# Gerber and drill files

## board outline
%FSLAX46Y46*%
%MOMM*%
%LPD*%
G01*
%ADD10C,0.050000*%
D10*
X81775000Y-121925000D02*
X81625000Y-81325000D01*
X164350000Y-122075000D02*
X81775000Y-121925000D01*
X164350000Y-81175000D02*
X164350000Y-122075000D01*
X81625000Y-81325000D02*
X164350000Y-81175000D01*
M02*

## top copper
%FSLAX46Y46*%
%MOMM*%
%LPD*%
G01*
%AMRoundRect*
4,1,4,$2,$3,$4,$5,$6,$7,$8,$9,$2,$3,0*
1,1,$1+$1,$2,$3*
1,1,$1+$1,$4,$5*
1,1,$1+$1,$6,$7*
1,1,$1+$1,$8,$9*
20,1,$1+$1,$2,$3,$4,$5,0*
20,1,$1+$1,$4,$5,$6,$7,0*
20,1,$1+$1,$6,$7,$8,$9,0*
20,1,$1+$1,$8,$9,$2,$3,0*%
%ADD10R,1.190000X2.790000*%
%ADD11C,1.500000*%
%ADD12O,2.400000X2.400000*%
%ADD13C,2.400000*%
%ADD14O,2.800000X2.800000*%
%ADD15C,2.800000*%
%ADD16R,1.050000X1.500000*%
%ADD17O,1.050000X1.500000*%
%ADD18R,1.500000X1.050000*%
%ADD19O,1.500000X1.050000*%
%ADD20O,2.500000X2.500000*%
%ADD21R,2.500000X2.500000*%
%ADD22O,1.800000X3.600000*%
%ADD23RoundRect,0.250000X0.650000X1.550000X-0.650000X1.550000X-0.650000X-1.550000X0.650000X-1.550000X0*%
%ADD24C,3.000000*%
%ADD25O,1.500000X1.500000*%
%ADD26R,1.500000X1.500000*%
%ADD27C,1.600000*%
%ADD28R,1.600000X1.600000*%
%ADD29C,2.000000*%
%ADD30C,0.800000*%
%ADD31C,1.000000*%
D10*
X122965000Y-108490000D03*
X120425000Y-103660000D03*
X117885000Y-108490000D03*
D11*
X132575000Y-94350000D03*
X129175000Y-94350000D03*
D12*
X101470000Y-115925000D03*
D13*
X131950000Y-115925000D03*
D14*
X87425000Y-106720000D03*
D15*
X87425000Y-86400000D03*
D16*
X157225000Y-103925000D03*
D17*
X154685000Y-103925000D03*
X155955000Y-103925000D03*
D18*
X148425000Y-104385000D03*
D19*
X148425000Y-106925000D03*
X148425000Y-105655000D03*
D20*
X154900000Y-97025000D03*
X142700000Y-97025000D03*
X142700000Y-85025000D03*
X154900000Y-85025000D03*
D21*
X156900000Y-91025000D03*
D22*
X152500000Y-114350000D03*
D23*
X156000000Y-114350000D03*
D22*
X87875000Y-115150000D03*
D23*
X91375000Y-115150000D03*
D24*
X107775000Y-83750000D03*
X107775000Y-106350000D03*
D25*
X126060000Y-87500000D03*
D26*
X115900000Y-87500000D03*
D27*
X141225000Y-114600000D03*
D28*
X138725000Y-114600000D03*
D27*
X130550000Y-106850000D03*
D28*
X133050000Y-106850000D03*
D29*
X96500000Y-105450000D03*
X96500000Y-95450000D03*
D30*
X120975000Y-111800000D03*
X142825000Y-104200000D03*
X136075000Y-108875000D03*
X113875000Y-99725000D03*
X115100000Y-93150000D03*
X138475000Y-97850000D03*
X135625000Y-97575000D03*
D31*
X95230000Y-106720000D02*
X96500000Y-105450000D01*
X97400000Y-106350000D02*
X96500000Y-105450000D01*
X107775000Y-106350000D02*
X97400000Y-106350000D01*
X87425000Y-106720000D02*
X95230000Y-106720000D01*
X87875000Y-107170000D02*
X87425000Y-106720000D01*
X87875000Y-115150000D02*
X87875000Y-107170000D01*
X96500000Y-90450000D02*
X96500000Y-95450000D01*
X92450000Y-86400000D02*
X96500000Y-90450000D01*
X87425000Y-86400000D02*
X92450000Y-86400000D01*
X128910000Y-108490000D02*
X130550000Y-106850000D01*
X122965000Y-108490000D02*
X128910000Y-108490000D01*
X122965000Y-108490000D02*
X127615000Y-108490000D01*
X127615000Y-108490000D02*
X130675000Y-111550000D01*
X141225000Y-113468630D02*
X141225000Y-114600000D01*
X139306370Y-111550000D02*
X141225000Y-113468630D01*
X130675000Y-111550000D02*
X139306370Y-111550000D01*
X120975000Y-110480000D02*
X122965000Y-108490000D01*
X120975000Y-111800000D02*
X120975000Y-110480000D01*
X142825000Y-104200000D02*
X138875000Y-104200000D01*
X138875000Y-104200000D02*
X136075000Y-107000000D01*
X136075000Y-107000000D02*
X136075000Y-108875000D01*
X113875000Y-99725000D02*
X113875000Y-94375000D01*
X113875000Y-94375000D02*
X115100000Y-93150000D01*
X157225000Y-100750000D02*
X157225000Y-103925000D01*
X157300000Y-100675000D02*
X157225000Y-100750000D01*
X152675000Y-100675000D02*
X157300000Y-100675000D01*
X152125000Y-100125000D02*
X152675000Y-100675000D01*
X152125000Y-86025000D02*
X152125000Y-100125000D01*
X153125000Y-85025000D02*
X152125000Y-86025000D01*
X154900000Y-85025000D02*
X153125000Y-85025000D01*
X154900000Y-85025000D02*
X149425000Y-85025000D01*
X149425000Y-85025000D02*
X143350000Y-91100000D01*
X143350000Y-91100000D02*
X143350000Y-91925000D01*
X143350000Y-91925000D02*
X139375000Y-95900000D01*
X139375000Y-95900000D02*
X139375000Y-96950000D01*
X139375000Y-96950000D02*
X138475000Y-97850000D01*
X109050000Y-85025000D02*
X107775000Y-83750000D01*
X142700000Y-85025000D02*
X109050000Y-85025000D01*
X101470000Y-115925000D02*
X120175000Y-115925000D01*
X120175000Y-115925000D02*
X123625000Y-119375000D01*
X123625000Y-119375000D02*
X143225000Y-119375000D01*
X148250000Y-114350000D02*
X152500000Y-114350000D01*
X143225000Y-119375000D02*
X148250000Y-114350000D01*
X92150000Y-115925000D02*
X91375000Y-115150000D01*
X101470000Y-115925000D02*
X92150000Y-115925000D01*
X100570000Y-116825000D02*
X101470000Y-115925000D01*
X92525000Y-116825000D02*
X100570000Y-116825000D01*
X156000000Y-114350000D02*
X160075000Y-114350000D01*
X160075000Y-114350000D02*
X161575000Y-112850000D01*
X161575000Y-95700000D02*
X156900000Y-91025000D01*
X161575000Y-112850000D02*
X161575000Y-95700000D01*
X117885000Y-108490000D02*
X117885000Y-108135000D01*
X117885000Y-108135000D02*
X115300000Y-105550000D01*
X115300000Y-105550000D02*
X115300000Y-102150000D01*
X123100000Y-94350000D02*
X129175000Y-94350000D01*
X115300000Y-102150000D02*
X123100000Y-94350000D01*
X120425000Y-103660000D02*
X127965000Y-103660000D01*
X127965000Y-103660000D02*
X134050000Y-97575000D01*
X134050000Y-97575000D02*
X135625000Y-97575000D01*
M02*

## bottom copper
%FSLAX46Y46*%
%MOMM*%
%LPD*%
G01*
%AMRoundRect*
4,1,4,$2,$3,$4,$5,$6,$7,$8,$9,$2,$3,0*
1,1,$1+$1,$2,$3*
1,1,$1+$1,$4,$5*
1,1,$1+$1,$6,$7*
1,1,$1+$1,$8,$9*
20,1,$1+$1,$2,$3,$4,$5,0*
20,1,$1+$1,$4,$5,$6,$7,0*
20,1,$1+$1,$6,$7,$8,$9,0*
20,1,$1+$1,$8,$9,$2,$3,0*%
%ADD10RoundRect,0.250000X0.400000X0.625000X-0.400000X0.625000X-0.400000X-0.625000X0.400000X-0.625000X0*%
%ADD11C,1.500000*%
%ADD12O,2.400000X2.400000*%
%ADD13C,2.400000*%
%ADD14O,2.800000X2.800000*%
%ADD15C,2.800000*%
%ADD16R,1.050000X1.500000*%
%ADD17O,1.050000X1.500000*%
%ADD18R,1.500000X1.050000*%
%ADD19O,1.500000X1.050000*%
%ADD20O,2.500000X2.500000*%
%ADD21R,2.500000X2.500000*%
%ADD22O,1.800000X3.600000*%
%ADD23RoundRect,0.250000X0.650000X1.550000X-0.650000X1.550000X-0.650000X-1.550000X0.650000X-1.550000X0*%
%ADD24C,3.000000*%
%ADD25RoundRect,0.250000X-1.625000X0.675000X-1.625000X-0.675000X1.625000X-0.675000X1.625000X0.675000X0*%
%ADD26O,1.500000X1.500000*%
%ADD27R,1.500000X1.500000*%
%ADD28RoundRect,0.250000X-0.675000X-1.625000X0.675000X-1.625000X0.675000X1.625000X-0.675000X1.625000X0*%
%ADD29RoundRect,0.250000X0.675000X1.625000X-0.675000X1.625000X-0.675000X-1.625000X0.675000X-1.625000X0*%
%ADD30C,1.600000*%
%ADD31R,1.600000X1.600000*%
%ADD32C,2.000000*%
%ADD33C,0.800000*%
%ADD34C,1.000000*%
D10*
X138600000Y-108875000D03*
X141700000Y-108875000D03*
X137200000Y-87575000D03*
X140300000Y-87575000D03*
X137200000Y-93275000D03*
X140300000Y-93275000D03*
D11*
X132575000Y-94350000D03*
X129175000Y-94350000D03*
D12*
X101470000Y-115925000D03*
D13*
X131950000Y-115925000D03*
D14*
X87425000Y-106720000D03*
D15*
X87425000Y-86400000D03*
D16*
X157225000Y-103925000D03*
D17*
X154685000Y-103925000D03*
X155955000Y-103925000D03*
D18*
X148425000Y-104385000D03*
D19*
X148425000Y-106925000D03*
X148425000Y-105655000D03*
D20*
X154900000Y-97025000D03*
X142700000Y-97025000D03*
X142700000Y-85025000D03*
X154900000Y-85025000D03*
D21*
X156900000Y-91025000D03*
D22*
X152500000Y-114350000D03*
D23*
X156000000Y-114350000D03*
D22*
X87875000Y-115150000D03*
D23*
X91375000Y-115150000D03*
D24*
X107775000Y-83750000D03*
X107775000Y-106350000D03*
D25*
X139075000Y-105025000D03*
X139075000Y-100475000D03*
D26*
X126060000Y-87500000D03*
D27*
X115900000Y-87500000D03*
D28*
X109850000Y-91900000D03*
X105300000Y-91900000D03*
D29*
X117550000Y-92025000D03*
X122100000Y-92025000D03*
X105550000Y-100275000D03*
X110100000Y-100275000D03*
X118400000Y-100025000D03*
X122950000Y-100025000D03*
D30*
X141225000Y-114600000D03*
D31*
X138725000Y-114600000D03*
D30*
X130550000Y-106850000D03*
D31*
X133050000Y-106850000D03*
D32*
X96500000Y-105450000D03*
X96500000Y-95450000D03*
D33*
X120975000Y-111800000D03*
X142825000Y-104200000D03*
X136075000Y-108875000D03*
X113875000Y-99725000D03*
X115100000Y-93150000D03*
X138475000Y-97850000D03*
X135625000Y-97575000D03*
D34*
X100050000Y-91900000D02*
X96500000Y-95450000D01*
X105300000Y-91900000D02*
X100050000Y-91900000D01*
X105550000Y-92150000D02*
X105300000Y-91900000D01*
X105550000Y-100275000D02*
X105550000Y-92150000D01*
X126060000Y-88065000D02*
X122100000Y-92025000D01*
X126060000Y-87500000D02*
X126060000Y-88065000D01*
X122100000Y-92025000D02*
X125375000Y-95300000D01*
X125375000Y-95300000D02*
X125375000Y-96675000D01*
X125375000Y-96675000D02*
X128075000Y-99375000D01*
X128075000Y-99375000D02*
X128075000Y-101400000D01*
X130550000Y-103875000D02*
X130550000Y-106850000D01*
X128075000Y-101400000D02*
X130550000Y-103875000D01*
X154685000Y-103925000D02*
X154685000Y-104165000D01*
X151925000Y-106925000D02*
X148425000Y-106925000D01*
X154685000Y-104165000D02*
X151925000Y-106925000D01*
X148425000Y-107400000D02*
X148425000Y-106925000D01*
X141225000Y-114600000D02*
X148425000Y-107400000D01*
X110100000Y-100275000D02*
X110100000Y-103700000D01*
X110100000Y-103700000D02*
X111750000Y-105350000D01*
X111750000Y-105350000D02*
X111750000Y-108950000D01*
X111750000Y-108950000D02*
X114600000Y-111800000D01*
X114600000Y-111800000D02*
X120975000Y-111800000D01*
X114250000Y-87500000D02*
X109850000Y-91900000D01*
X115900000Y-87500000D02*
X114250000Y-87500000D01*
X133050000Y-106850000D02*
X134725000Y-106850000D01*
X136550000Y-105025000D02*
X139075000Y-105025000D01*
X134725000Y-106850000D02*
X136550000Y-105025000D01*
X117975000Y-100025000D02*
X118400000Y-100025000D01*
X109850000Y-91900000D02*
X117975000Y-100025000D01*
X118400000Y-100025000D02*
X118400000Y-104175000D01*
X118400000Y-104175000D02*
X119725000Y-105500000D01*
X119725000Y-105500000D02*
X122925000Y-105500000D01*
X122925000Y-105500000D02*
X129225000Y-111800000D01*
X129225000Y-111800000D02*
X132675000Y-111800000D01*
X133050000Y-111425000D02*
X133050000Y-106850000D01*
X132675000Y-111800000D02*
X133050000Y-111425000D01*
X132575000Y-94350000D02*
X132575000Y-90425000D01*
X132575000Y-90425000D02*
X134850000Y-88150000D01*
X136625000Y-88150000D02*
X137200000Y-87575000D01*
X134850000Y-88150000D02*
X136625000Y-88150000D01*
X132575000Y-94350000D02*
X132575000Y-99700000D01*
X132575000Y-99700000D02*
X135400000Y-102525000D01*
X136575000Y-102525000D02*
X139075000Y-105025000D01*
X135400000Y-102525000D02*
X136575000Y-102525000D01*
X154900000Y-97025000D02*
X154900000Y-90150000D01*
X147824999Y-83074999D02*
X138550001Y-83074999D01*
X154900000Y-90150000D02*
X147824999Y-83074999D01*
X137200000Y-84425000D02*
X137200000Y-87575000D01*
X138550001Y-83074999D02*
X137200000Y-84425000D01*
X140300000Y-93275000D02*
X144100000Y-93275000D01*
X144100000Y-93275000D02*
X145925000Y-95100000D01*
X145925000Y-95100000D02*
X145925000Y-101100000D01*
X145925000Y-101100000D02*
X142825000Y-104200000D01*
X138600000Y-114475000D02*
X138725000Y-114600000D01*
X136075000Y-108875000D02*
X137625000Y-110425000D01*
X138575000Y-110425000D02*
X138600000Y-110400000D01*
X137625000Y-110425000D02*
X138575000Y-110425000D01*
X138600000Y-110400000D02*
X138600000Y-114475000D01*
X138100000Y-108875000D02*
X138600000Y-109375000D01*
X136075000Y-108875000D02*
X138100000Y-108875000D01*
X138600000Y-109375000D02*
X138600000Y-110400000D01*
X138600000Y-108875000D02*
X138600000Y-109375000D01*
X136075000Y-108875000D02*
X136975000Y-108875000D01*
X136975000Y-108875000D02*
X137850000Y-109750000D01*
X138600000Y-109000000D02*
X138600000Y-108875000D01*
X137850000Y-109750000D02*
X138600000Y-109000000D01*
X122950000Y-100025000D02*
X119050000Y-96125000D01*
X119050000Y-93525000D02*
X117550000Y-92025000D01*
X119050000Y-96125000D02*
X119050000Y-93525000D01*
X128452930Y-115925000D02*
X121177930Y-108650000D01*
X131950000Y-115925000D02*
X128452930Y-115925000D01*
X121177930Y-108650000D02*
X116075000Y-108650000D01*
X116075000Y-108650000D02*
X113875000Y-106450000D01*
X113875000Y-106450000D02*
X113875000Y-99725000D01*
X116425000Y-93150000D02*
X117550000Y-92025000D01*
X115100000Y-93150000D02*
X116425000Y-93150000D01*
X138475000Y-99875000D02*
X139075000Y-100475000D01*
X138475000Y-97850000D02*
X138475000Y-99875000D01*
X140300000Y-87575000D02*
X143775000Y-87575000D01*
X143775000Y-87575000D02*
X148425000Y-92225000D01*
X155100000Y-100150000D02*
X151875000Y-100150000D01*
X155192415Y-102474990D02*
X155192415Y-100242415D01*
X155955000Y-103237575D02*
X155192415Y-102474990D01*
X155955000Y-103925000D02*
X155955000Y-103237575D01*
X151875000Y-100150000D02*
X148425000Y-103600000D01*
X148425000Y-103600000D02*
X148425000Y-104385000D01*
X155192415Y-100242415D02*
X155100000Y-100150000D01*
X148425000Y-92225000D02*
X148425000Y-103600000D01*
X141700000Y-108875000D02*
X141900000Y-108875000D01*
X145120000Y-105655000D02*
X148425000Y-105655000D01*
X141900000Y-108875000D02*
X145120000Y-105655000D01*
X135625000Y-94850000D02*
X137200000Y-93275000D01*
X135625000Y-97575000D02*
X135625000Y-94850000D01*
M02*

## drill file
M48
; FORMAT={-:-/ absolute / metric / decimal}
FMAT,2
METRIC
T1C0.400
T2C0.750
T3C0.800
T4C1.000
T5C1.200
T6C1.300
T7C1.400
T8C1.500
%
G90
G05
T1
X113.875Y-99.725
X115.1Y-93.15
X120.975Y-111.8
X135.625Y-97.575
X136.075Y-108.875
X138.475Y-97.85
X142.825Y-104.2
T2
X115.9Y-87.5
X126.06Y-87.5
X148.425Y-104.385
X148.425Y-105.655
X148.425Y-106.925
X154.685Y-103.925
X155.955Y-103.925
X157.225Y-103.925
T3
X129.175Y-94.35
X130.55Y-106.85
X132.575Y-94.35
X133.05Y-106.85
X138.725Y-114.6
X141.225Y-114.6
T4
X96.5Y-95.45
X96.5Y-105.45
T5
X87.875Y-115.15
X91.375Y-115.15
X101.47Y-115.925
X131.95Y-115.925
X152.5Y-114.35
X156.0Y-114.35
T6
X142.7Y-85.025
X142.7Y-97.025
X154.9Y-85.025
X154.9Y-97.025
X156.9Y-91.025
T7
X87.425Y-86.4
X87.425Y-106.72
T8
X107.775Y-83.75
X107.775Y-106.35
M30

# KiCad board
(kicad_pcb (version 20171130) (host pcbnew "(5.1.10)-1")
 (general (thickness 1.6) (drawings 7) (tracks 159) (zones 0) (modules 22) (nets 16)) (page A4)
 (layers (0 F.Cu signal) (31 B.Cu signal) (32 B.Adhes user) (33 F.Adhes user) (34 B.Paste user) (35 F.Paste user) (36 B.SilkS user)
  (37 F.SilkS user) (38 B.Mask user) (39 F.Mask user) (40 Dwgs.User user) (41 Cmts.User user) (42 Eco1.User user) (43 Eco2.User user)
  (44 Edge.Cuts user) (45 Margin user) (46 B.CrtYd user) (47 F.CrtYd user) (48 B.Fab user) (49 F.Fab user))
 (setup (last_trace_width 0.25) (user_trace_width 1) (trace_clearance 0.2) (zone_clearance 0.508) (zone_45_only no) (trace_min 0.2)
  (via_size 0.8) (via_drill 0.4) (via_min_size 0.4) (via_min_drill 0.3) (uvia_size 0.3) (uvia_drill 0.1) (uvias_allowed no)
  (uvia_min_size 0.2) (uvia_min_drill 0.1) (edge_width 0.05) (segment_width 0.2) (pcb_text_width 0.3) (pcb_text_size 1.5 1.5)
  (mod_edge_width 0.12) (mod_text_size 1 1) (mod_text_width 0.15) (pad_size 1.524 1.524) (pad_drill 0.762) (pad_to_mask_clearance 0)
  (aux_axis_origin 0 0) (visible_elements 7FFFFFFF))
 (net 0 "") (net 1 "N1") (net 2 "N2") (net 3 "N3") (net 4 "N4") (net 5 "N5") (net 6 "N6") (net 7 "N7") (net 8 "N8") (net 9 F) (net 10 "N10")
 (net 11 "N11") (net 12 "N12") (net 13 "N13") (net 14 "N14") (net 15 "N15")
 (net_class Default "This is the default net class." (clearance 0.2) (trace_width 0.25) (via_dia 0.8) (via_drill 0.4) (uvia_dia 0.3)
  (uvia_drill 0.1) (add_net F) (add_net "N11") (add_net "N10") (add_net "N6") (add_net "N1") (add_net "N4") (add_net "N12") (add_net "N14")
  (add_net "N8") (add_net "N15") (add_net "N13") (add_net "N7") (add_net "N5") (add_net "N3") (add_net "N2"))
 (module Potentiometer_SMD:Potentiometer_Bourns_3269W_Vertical (layer F.Cu) (at 120.425 106.075 180)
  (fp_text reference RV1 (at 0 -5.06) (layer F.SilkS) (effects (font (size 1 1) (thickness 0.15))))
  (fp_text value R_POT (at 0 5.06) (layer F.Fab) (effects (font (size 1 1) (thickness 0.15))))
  (pad 3 smd rect (at -2.54 -2.415 180) (size 1.19 2.79) (layers F.Cu F.Paste F.Mask) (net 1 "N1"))
  (pad 2 smd rect (at 0 2.415 180) (size 1.19 2.79) (layers F.Cu F.Paste F.Mask) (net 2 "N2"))
  (pad 1 smd rect (at 2.54 -2.415 180) (size 1.19 2.79) (layers F.Cu F.Paste F.Mask) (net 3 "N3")))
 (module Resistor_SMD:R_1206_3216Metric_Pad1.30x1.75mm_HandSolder (layer B.Cu) (at 140.15 108.875 180)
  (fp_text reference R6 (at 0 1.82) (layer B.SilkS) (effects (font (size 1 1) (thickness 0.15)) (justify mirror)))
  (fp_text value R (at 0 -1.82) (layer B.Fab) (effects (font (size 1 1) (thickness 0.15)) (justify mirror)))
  (pad 2 smd roundrect (at 1.55 0 180) (size 1.3 1.75) (layers B.Cu B.Paste B.Mask) (roundrect_rratio 0.192308) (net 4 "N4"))
  (pad 1 smd roundrect (at -1.55 0 180) (size 1.3 1.75) (layers B.Cu B.Paste B.Mask) (roundrect_rratio 0.192308) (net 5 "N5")))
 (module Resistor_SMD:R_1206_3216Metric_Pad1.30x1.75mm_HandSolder (layer B.Cu) (at 138.75 87.575 180)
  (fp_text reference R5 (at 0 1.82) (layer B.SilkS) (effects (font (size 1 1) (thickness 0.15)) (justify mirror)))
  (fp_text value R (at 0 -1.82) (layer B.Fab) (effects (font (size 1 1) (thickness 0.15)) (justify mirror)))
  (pad 2 smd roundrect (at 1.55 0 180) (size 1.3 1.75) (layers B.Cu B.Paste B.Mask) (roundrect_rratio 0.192308) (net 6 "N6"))
  (pad 1 smd roundrect (at -1.55 0 180) (size 1.3 1.75) (layers B.Cu B.Paste B.Mask) (roundrect_rratio 0.192308) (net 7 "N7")))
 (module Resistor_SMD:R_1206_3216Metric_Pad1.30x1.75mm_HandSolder (layer B.Cu) (at 138.75 93.275 180)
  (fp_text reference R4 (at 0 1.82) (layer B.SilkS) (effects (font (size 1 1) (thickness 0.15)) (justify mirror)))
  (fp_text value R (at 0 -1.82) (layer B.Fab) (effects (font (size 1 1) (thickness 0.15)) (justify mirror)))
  (pad 2 smd roundrect (at 1.55 0 180) (size 1.3 1.75) (layers B.Cu B.Paste B.Mask) (roundrect_rratio 0.192308) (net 2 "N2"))
  (pad 1 smd roundrect (at -1.55 0 180) (size 1.3 1.75) (layers B.Cu B.Paste B.Mask) (roundrect_rratio 0.192308) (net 4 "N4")))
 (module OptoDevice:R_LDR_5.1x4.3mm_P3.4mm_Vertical (layer F.Cu) (at 129.175 94.35)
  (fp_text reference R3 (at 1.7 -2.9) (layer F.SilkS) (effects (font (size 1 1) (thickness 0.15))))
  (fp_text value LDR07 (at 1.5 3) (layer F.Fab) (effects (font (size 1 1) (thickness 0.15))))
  (pad 2 thru_hole circle (at 3.4 0) (size 1.5 1.5) (drill 0.8) (layers *.Cu *.Mask) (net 6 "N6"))
  (pad 1 thru_hole circle (at 0 0) (size 1.5 1.5) (drill 0.8) (layers *.Cu *.Mask) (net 3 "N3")))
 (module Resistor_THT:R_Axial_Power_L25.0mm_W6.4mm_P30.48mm (layer F.Cu) (at 131.95 115.925 180)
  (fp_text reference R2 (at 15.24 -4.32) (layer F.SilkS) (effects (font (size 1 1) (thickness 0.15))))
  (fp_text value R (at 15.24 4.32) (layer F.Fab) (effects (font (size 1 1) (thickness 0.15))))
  (pad 2 thru_hole oval (at 30.48 0 180) (size 2.4 2.4) (drill 1.2) (layers *.Cu *.Mask) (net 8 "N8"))
  (pad 1 thru_hole circle (at 0 0 180) (size 2.4 2.4) (drill 1.2) (layers *.Cu *.Mask) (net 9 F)))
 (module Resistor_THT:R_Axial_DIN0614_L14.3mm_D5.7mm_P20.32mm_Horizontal (layer F.Cu) (at 87.425 86.4 270)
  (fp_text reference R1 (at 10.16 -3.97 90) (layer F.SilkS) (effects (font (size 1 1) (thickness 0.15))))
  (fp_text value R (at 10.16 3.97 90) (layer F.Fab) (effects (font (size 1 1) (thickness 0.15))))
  (pad 2 thru_hole oval (at 20.32 0 270) (size 2.8 2.8) (drill 1.4) (layers *.Cu *.Mask) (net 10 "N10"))
  (pad 1 thru_hole circle (at 0 0 270) (size 2.8 2.8) (drill 1.4) (layers *.Cu *.Mask) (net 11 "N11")))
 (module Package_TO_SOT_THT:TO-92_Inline (layer F.Cu) (at 157.225 103.925 180)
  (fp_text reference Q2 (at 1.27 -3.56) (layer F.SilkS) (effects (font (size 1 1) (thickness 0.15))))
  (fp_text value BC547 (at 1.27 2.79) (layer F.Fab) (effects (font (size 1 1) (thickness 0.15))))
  (pad 1 thru_hole rect (at 0 0 180) (size 1.05 1.5) (drill 0.75) (layers *.Cu *.Mask) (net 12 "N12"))
  (pad 3 thru_hole oval (at 2.54 0 180) (size 1.05 1.5) (drill 0.75) (layers *.Cu *.Mask) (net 1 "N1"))
  (pad 2 thru_hole oval (at 1.27 0 180) (size 1.05 1.5) (drill 0.75) (layers *.Cu *.Mask) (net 7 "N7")))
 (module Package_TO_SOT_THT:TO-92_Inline (layer F.Cu) (at 148.425 104.385 270)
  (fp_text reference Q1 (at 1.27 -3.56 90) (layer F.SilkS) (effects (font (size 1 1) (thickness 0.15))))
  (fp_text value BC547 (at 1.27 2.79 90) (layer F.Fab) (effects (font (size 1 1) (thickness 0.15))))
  (pad 1 thru_hole rect (at 0 0 270) (size 1.05 1.5) (drill 0.75) (layers *.Cu *.Mask) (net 7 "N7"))
  (pad 3 thru_hole oval (at 2.54 0 270) (size 1.05 1.5) (drill 0.75) (layers *.Cu *.Mask) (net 1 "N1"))
  (pad 2 thru_hole oval (at 1.27 0 270) (size 1.05 1.5) (drill 0.75) (layers *.Cu *.Mask) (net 5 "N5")))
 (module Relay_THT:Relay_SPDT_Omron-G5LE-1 (layer F.Cu) (at 156.9 91.025 270)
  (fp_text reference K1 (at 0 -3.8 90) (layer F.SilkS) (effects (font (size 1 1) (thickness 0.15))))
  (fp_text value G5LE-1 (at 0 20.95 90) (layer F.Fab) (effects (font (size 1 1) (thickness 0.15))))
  (pad 5 thru_hole oval (at 6 2 270) (size 2.5 2.5) (drill 1.3) (layers *.Cu *.Mask) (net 6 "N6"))
  (pad 4 thru_hole oval (at 6 14.2 270) (size 2.5 2.5) (drill 1.3) (layers *.Cu *.Mask) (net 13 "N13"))
  (pad 3 thru_hole oval (at -6 14.2 270) (size 2.5 2.5) (drill 1.3) (layers *.Cu *.Mask) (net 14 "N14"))
  (pad 2 thru_hole oval (at -6 2 270) (size 2.5 2.5) (drill 1.3) (layers *.Cu *.Mask) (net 12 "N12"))
  (pad 1 thru_hole rect (at 0 0 270) (size 2.5 2.5) (drill 1.3) (layers *.Cu *.Mask) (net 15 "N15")))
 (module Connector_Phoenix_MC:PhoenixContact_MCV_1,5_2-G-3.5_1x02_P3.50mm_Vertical (layer F.Cu) (at 156 114.35 180)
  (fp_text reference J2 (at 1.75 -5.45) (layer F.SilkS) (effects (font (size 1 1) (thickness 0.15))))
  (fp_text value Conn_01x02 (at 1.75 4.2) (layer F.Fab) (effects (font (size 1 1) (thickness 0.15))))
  (pad 2 thru_hole oval (at 3.5 0 180) (size 1.8 3.6) (drill 1.2) (layers *.Cu *.Mask) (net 8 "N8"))
  (pad 1 thru_hole roundrect (at 0 0 180) (size 1.8 3.6) (drill 1.2) (layers *.Cu *.Mask) (roundrect_rratio 0.138889) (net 15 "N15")))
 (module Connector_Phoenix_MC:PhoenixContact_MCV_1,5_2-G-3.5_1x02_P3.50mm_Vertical (layer F.Cu) (at 91.375 115.15 180)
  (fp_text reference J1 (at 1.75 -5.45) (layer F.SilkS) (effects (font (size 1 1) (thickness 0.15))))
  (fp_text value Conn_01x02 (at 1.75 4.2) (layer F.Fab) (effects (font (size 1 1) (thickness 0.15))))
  (pad 2 thru_hole oval (at 3.5 0 180) (size 1.8 3.6) (drill 1.2) (layers *.Cu *.Mask) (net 10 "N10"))
  (pad 1 thru_hole roundrect (at 0 0 180) (size 1.8 3.6) (drill 1.2) (layers *.Cu *.Mask) (roundrect_rratio 0.138889) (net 8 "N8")))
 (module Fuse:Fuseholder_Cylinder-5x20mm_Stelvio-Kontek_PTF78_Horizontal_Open (layer F.Cu) (at 107.775 83.75 270)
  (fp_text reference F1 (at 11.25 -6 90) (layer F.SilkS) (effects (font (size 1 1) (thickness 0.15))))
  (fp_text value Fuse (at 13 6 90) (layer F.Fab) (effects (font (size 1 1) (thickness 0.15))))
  (pad 1 thru_hole circle (at 0 0 270) (size 3 3) (drill 1.5) (layers *.Cu *.Mask) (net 14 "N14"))
  (pad 2 thru_hole circle (at 22.6 0 270) (size 3 3) (drill 1.5) (layers *.Cu *.Mask) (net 10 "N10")))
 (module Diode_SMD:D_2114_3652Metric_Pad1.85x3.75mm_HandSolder (layer B.Cu) (at 139.075 102.75 270)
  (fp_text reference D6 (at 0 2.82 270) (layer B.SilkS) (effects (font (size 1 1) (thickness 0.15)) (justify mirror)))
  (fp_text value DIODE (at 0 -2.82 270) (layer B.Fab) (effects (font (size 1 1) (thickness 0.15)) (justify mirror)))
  (pad 2 smd roundrect (at 2.275 0 270) (size 1.85 3.75) (layers B.Cu B.Paste B.Mask) (roundrect_rratio 0.135135) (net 6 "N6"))
  (pad 1 smd roundrect (at -2.275 0 270) (size 1.85 3.75) (layers B.Cu B.Paste B.Mask) (roundrect_rratio 0.135135) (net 12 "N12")))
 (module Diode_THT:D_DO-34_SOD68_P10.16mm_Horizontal (layer F.Cu) (at 115.9 87.5)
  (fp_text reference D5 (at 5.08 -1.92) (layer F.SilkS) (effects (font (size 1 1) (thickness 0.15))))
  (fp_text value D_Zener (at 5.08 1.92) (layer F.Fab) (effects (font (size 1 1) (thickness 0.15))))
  (pad 2 thru_hole oval (at 10.16 0) (size 1.5 1.5) (drill 0.75) (layers *.Cu *.Mask) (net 1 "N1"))
  (pad 1 thru_hole rect (at 0 0) (size 1.5 1.5) (drill 0.75) (layers *.Cu *.Mask) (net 6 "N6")))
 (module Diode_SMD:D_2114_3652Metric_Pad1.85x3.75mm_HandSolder (layer B.Cu) (at 107.575 91.9)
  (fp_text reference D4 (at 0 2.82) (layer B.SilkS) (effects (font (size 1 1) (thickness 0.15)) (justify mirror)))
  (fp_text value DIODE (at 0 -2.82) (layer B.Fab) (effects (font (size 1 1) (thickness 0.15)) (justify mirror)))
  (pad 2 smd roundrect (at 2.275 0) (size 1.85 3.75) (layers B.Cu B.Paste B.Mask) (roundrect_rratio 0.135135) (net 6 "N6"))
  (pad 1 smd roundrect (at -2.275 0) (size 1.85 3.75) (layers B.Cu B.Paste B.Mask) (roundrect_rratio 0.135135) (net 11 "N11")))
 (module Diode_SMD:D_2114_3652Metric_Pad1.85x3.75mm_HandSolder (layer B.Cu) (at 119.825 92.025 180)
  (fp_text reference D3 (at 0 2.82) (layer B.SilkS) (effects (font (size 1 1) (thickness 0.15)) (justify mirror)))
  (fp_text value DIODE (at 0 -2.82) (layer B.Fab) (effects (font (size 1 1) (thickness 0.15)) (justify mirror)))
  (pad 2 smd roundrect (at 2.275 0 180) (size 1.85 3.75) (layers B.Cu B.Paste B.Mask) (roundrect_rratio 0.135135) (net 9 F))
  (pad 1 smd roundrect (at -2.275 0 180) (size 1.85 3.75) (layers B.Cu B.Paste B.Mask) (roundrect_rratio 0.135135) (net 1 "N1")))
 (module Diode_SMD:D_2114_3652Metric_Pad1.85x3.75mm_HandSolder (layer B.Cu) (at 107.825 100.275 180)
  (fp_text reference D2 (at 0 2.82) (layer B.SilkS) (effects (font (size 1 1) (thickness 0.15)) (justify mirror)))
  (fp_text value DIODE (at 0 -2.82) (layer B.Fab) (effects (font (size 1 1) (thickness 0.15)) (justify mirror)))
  (pad 2 smd roundrect (at 2.275 0 180) (size 1.85 3.75) (layers B.Cu B.Paste B.Mask) (roundrect_rratio 0.135135) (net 11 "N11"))
  (pad 1 smd roundrect (at -2.275 0 180) (size 1.85 3.75) (layers B.Cu B.Paste B.Mask) (roundrect_rratio 0.135135) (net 1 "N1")))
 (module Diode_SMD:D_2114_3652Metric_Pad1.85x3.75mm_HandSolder (layer B.Cu) (at 120.675 100.025 180)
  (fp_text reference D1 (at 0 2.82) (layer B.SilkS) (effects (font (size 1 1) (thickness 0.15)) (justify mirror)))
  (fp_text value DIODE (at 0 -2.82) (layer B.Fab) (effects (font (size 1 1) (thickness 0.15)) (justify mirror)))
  (pad 2 smd roundrect (at 2.275 0 180) (size 1.85 3.75) (layers B.Cu B.Paste B.Mask) (roundrect_rratio 0.135135) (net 6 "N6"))
  (pad 1 smd roundrect (at -2.275 0 180) (size 1.85 3.75) (layers B.Cu B.Paste B.Mask) (roundrect_rratio 0.135135) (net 9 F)))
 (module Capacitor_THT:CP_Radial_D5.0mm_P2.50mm (layer F.Cu) (at 138.725 114.6)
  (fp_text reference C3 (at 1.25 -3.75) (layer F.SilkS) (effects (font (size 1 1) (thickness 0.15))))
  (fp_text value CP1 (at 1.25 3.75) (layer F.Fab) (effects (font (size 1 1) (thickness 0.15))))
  (pad 2 thru_hole circle (at 2.5 0) (size 1.6 1.6) (drill 0.8) (layers *.Cu *.Mask) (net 1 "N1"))
  (pad 1 thru_hole rect (at 0 0) (size 1.6 1.6) (drill 0.8) (layers *.Cu *.Mask) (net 4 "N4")))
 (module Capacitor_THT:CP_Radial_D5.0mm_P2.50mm (layer F.Cu) (at 133.05 106.85 180)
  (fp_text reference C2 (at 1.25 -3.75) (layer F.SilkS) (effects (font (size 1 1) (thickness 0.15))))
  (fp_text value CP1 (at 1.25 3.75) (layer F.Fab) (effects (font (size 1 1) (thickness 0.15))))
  (pad 2 thru_hole circle (at 2.5 0 180) (size 1.6 1.6) (drill 0.8) (layers *.Cu *.Mask) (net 1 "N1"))
  (pad 1 thru_hole rect (at 0 0 180) (size 1.6 1.6) (drill 0.8) (layers *.Cu *.Mask) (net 6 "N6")))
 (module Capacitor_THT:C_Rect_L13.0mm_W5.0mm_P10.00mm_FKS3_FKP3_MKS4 (layer F.Cu) (at 96.5 95.45 270)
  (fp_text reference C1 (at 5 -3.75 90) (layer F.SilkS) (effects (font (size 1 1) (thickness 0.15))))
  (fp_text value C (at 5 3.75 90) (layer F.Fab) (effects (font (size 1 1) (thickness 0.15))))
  (pad 2 thru_hole circle (at 10 0 270) (size 2 2) (drill 1) (layers *.Cu *.Mask) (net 10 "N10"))
  (pad 1 thru_hole circle (at 0 0 270) (size 2 2) (drill 1) (layers *.Cu *.Mask) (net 11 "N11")))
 (gr_line (start 81.775 121.925) (end 81.625 81.325) (layer Edge.Cuts) (width 0.05))
 (gr_line (start 164.35 122.075) (end 81.775 121.925) (layer Edge.Cuts) (width 0.05))
 (gr_line (start 164.35 81.175) (end 164.35 122.075) (layer Edge.Cuts) (width 0.05))
 (gr_line (start 81.625 81.325) (end 164.35 81.175) (layer Edge.Cuts) (width 0.05))
 (segment (start 95.23 106.72) (end 96.5 105.45) (width 1) (layer F.Cu) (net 10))
 (segment (start 97.4 106.35) (end 96.5 105.45) (width 1) (layer F.Cu) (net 10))
 (segment (start 107.775 106.35) (end 97.4 106.35) (width 1) (layer F.Cu) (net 10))
 (segment (start 87.425 106.72) (end 95.23 106.72) (width 1) (layer F.Cu) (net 10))
 (segment (start 87.875 107.17) (end 87.425 106.72) (width 1) (layer F.Cu) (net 10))
 (segment (start 87.875 115.15) (end 87.875 107.17) (width 1) (layer F.Cu) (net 10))
 (segment (start 100.05 91.9) (end 96.5 95.45) (width 1) (layer B.Cu) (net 11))
 (segment (start 105.3 91.9) (end 100.05 91.9) (width 1) (layer B.Cu) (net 11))
 (segment (start 105.55 92.15) (end 105.3 91.9) (width 1) (layer B.Cu) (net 11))
 (segment (start 105.55 100.275) (end 105.55 92.15) (width 1) (layer B.Cu) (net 11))
 (segment (start 96.5 90.45) (end 96.5 95.45) (width 1) (layer F.Cu) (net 11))
 (segment (start 92.45 86.4) (end 96.5 90.45) (width 1) (layer F.Cu) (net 11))
 (segment (start 87.425 86.4) (end 92.45 86.4) (width 1) (layer F.Cu) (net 11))
 (segment (start 128.91 108.49) (end 130.55 106.85) (width 1) (layer F.Cu) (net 1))
 (segment (start 122.965 108.49) (end 128.91 108.49) (width 1) (layer F.Cu) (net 1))
 (segment (start 126.06 88.065) (end 122.1 92.025) (width 1) (layer B.Cu) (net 1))
 (segment (start 126.06 87.5) (end 126.06 88.065) (width 1) (layer B.Cu) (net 1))
 (segment (start 122.1 92.025) (end 125.375 95.3) (width 1) (layer B.Cu) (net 1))
 (segment (start 125.375 95.3) (end 125.375 96.675) (width 1) (layer B.Cu) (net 1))
 (segment (start 125.375 96.675) (end 128.075 99.375) (width 1) (layer B.Cu) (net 1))
 (segment (start 128.075 99.375) (end 128.075 101.4) (width 1) (layer B.Cu) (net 1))
 (segment (start 130.55 103.875) (end 130.55 106.85) (width 1) (layer B.Cu) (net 1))
 (segment (start 128.075 101.4) (end 130.55 103.875) (width 1) (layer B.Cu) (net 1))
 (segment (start 122.965 108.49) (end 127.615 108.49) (width 1) (layer F.Cu) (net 1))
 (segment (start 127.615 108.49) (end 130.675 111.55) (width 1) (layer F.Cu) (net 1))
 (segment (start 141.225 113.46863) (end 141.225 114.6) (width 1) (layer F.Cu) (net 1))
 (segment (start 139.30637 111.55) (end 141.225 113.46863) (width 1) (layer F.Cu) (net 1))
 (segment (start 130.675 111.55) (end 139.30637 111.55) (width 1) (layer F.Cu) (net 1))
 (segment (start 154.685 103.925) (end 154.685 104.165) (width 1) (layer B.Cu) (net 1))
 (segment (start 151.925 106.925) (end 148.425 106.925) (width 1) (layer B.Cu) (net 1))
 (segment (start 154.685 104.165) (end 151.925 106.925) (width 1) (layer B.Cu) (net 1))
 (segment (start 148.425 107.4) (end 148.425 106.925) (width 1) (layer B.Cu) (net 1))
 (segment (start 141.225 114.6) (end 148.425 107.4) (width 1) (layer B.Cu) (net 1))
 (segment (start 110.1 100.275) (end 110.1 103.7) (width 1) (layer B.Cu) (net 1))
 (segment (start 110.1 103.7) (end 111.75 105.35) (width 1) (layer B.Cu) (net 1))
 (segment (start 111.75 105.35) (end 111.75 108.95) (width 1) (layer B.Cu) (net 1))
 (segment (start 111.75 108.95) (end 114.6 111.8) (width 1) (layer B.Cu) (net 1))
 (segment (start 114.6 111.8) (end 120.975 111.8) (width 1) (layer B.Cu) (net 1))
 (via (at 120.975 111.8) (size 0.8) (drill 0.4) (layers F.Cu B.Cu) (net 1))
 (segment (start 120.975 110.48) (end 122.965 108.49) (width 1) (layer F.Cu) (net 1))
 (segment (start 120.975 111.8) (end 120.975 110.48) (width 1) (layer F.Cu) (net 1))
 (segment (start 114.25 87.5) (end 109.85 91.9) (width 1) (layer B.Cu) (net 6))
 (segment (start 115.9 87.5) (end 114.25 87.5) (width 1) (layer B.Cu) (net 6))
 (segment (start 133.05 106.85) (end 134.725 106.85) (width 1) (layer B.Cu) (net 6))
 (segment (start 136.55 105.025) (end 139.075 105.025) (width 1) (layer B.Cu) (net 6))
 (segment (start 134.725 106.85) (end 136.55 105.025) (width 1) (layer B.Cu) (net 6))
 (segment (start 117.975 100.025) (end 118.4 100.025) (width 1) (layer B.Cu) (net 6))
 (segment (start 109.85 91.9) (end 117.975 100.025) (width 1) (layer B.Cu) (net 6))
 (segment (start 118.4 100.025) (end 118.4 104.175) (width 1) (layer B.Cu) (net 6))
 (segment (start 118.4 104.175) (end 119.725 105.5) (width 1) (layer B.Cu) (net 6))
 (segment (start 119.725 105.5) (end 122.925 105.5) (width 1) (layer B.Cu) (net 6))
 (segment (start 122.925 105.5) (end 129.225 111.8) (width 1) (layer B.Cu) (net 6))
 (segment (start 129.225 111.8) (end 132.675 111.8) (width 1) (layer B.Cu) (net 6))
 (segment (start 133.05 111.425) (end 133.05 106.85) (width 1) (layer B.Cu) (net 6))
 (segment (start 132.675 111.8) (end 133.05 111.425) (width 1) (layer B.Cu) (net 6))
 (segment (start 132.575 94.35) (end 132.575 90.425) (width 1) (layer B.Cu) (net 6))
 (segment (start 132.575 90.425) (end 134.85 88.15) (width 1) (layer B.Cu) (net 6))
 (segment (start 136.625 88.15) (end 137.2 87.575) (width 1) (layer B.Cu) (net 6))
 (segment (start 134.85 88.15) (end 136.625 88.15) (width 1) (layer B.Cu) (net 6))
 (segment (start 132.575 94.35) (end 132.575 99.7) (width 1) (layer B.Cu) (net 6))
 (segment (start 132.575 99.7) (end 135.4 102.525) (width 1) (layer B.Cu) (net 6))
 (segment (start 136.575 102.525) (end 139.075 105.025) (width 1) (layer B.Cu) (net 6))
 (segment (start 135.4 102.525) (end 136.575 102.525) (width 1) (layer B.Cu) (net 6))
 (segment (start 154.9 97.025) (end 154.9 90.15) (width 1) (layer B.Cu) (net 6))
 (segment (start 147.824999 83.074999) (end 138.550001 83.074999) (width 1) (layer B.Cu) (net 6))
 (segment (start 154.9 90.15) (end 147.824999 83.074999) (width 1) (layer B.Cu) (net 6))
 (segment (start 137.2 84.425) (end 137.2 87.575) (width 1) (layer B.Cu) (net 6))
 (segment (start 138.550001 83.074999) (end 137.2 84.425) (width 1) (layer B.Cu) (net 6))
 (segment (start 140.3 93.275) (end 144.1 93.275) (width 1) (layer B.Cu) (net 4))
 (segment (start 144.1 93.275) (end 145.925 95.1) (width 1) (layer B.Cu) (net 4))
 (segment (start 145.925 95.1) (end 145.925 101.1) (width 1) (layer B.Cu) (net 4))
 (segment (start 145.925 101.1) (end 142.825 104.2) (width 1) (layer B.Cu) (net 4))
 (via (at 142.825 104.2) (size 0.8) (drill 0.4) (layers F.Cu B.Cu) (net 4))
 (segment (start 142.825 104.2) (end 138.875 104.2) (width 1) (layer F.Cu) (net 4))
 (segment (start 138.875 104.2) (end 136.075 107) (width 1) (layer F.Cu) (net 4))
 (segment (start 136.075 107) (end 136.075 108.875) (width 1) (layer F.Cu) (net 4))
 (via (at 136.075 108.875) (size 0.8) (drill 0.4) (layers F.Cu B.Cu) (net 4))
 (segment (start 138.6 114.475) (end 138.725 114.6) (width 1) (layer B.Cu) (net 4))
 (segment (start 136.075 108.875) (end 137.625 110.425) (width 1) (layer B.Cu) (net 4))
 (segment (start 138.575 110.425) (end 138.6 110.4) (width 1) (layer B.Cu) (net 4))
 (segment (start 137.625 110.425) (end 138.575 110.425) (width 1) (layer B.Cu) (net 4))
 (segment (start 138.6 110.4) (end 138.6 114.475) (width 1) (layer B.Cu) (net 4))
 (segment (start 138.1 108.875) (end 138.6 109.375) (width 1) (layer B.Cu) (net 4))
 (segment (start 136.075 108.875) (end 138.1 108.875) (width 1) (layer B.Cu) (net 4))
 (segment (start 138.6 109.375) (end 138.6 110.4) (width 1) (layer B.Cu) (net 4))
 (segment (start 138.6 108.875) (end 138.6 109.375) (width 1) (layer B.Cu) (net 4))
 (segment (start 136.075 108.875) (end 136.975 108.875) (width 1) (layer B.Cu) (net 4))
 (segment (start 136.975 108.875) (end 137.85 109.75) (width 1) (layer B.Cu) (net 4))
 (segment (start 138.6 109) (end 138.6 108.875) (width 1) (layer B.Cu) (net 4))
 (segment (start 137.85 109.75) (end 138.6 109) (width 1) (layer B.Cu) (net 4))
 (segment (start 122.95 100.025) (end 119.05 96.125) (width 1) (layer B.Cu) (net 9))
 (segment (start 119.05 93.525) (end 117.55 92.025) (width 1) (layer B.Cu) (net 9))
 (segment (start 119.05 96.125) (end 119.05 93.525) (width 1) (layer B.Cu) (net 9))
 (segment (start 128.45293 115.925) (end 121.17793 108.65) (width 1) (layer B.Cu) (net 9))
 (segment (start 131.95 115.925) (end 128.45293 115.925) (width 1) (layer B.Cu) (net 9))
 (segment (start 121.17793 108.65) (end 116.075 108.65) (width 1) (layer B.Cu) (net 9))
 (segment (start 116.075 108.65) (end 113.875 106.45) (width 1) (layer B.Cu) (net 9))
 (segment (start 113.875 106.45) (end 113.875 99.725) (width 1) (layer B.Cu) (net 9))
 (via (at 113.875 99.725) (size 0.8) (drill 0.4) (layers F.Cu B.Cu) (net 9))
 (segment (start 113.875 99.725) (end 113.875 94.375) (width 1) (layer F.Cu) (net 9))
 (via (at 115.1 93.15) (size 0.8) (drill 0.4) (layers F.Cu B.Cu) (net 9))
 (segment (start 113.875 94.375) (end 115.1 93.15) (width 1) (layer F.Cu) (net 9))
 (segment (start 116.425 93.15) (end 117.55 92.025) (width 1) (layer B.Cu) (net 9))
 (segment (start 115.1 93.15) (end 116.425 93.15) (width 1) (layer B.Cu) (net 9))
 (segment (start 157.225 100.75) (end 157.225 103.925) (width 1) (layer F.Cu) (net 12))
 (segment (start 157.3 100.675) (end 157.225 100.75) (width 1) (layer F.Cu) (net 12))
 (segment (start 152.675 100.675) (end 157.3 100.675) (width 1) (layer F.Cu) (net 12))
 (segment (start 152.125 100.125) (end 152.675 100.675) (width 1) (layer F.Cu) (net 12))
 (segment (start 152.125 86.025) (end 152.125 100.125) (width 1) (layer F.Cu) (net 12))
 (segment (start 153.125 85.025) (end 152.125 86.025) (width 1) (layer F.Cu) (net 12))
 (segment (start 154.9 85.025) (end 153.125 85.025) (width 1) (layer F.Cu) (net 12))
 (segment (start 154.9 85.025) (end 149.425 85.025) (width 1) (layer F.Cu) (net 12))
 (segment (start 149.425 85.025) (end 143.35 91.1) (width 1) (layer F.Cu) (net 12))
 (segment (start 143.35 91.1) (end 143.35 91.925) (width 1) (layer F.Cu) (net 12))
 (segment (start 143.35 91.925) (end 139.375 95.9) (width 1) (layer F.Cu) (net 12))
 (segment (start 139.375 95.9) (end 139.375 96.95) (width 1) (layer F.Cu) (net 12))
 (via (at 138.475 97.85) (size 0.8) (drill 0.4) (layers F.Cu B.Cu) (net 12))
 (segment (start 139.375 96.95) (end 138.475 97.85) (width 1) (layer F.Cu) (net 12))
 (segment (start 138.475 99.875) (end 139.075 100.475) (width 1) (layer B.Cu) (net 12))
 (segment (start 138.475 97.85) (end 138.475 99.875) (width 1) (layer B.Cu) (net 12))
 (segment (start 109.05 85.025) (end 107.775 83.75) (width 1) (layer F.Cu) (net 14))
 (segment (start 142.7 85.025) (end 109.05 85.025) (width 1) (layer F.Cu) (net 14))
 (segment (start 101.47 115.925) (end 120.175 115.925) (width 1) (layer F.Cu) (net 8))
 (segment (start 120.175 115.925) (end 123.625 119.375) (width 1) (layer F.Cu) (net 8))
 (segment (start 123.625 119.375) (end 143.225 119.375) (width 1) (layer F.Cu) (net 8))
 (segment (start 148.25 114.35) (end 152.5 114.35) (width 1) (layer F.Cu) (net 8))
 (segment (start 143.225 119.375) (end 148.25 114.35) (width 1) (layer F.Cu) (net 8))
 (segment (start 92.15 115.925) (end 91.375 115.15) (width 1) (layer F.Cu) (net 8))
 (segment (start 101.47 115.925) (end 92.15 115.925) (width 1) (layer F.Cu) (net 8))
 (segment (start 100.57 116.825) (end 101.47 115.925) (width 1) (layer F.Cu) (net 8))
 (segment (start 92.525 116.825) (end 100.57 116.825) (width 1) (layer F.Cu) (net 8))
 (segment (start 156 114.35) (end 160.075 114.35) (width 1) (layer F.Cu) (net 15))
 (segment (start 160.075 114.35) (end 161.575 112.85) (width 1) (layer F.Cu) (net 15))
 (segment (start 161.575 95.7) (end 156.9 91.025) (width 1) (layer F.Cu) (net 15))
 (segment (start 161.575 112.85) (end 161.575 95.7) (width 1) (layer F.Cu) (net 15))
 (segment (start 140.3 87.575) (end 143.775 87.575) (width 1) (layer B.Cu) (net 7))
 (segment (start 143.775 87.575) (end 148.425 92.225) (width 1) (layer B.Cu) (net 7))
 (segment (start 155.1 100.15) (end 151.875 100.15) (width 1) (layer B.Cu) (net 7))
 (segment (start 155.192415 102.47499) (end 155.192415 100.242415) (width 1) (layer B.Cu) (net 7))
 (segment (start 155.955 103.237575) (end 155.192415 102.47499) (width 1) (layer B.Cu) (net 7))
 (segment (start 155.955 103.925) (end 155.955 103.237575) (width 1) (layer B.Cu) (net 7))
 (segment (start 151.875 100.15) (end 148.425 103.6) (width 1) (layer B.Cu) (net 7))
 (segment (start 148.425 103.6) (end 148.425 104.385) (width 1) (layer B.Cu) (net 7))
 (segment (start 155.192415 100.242415) (end 155.1 100.15) (width 1) (layer B.Cu) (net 7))
 (segment (start 148.425 92.225) (end 148.425 103.6) (width 1) (layer B.Cu) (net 7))
 (segment (start 141.7 108.875) (end 141.9 108.875) (width 1) (layer B.Cu) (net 5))
 (segment (start 145.12 105.655) (end 148.425 105.655) (width 1) (layer B.Cu) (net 5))
 (segment (start 141.9 108.875) (end 145.12 105.655) (width 1) (layer B.Cu) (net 5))
 (segment (start 117.885 108.49) (end 117.885 108.135) (width 1) (layer F.Cu) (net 3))
 (segment (start 117.885 108.135) (end 115.3 105.55) (width 1) (layer F.Cu) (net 3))
 (segment (start 115.3 105.55) (end 115.3 102.15) (width 1) (layer F.Cu) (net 3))
 (segment (start 123.1 94.35) (end 129.175 94.35) (width 1) (layer F.Cu) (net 3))
 (segment (start 115.3 102.15) (end 123.1 94.35) (width 1) (layer F.Cu) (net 3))
 (segment (start 120.425 103.66) (end 127.965 103.66) (width 1) (layer F.Cu) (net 2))
 (segment (start 127.965 103.66) (end 134.05 97.575) (width 1) (layer F.Cu) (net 2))
 (via (at 135.625 97.575) (size 0.8) (drill 0.4) (layers F.Cu B.Cu) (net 2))
 (segment (start 134.05 97.575) (end 135.625 97.575) (width 1) (layer F.Cu) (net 2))
 (segment (start 135.625 94.85) (end 137.2 93.275) (width 1) (layer B.Cu) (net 2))
 (segment (start 135.625 97.575) (end 135.625 94.85) (width 1) (layer B.Cu) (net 2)))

